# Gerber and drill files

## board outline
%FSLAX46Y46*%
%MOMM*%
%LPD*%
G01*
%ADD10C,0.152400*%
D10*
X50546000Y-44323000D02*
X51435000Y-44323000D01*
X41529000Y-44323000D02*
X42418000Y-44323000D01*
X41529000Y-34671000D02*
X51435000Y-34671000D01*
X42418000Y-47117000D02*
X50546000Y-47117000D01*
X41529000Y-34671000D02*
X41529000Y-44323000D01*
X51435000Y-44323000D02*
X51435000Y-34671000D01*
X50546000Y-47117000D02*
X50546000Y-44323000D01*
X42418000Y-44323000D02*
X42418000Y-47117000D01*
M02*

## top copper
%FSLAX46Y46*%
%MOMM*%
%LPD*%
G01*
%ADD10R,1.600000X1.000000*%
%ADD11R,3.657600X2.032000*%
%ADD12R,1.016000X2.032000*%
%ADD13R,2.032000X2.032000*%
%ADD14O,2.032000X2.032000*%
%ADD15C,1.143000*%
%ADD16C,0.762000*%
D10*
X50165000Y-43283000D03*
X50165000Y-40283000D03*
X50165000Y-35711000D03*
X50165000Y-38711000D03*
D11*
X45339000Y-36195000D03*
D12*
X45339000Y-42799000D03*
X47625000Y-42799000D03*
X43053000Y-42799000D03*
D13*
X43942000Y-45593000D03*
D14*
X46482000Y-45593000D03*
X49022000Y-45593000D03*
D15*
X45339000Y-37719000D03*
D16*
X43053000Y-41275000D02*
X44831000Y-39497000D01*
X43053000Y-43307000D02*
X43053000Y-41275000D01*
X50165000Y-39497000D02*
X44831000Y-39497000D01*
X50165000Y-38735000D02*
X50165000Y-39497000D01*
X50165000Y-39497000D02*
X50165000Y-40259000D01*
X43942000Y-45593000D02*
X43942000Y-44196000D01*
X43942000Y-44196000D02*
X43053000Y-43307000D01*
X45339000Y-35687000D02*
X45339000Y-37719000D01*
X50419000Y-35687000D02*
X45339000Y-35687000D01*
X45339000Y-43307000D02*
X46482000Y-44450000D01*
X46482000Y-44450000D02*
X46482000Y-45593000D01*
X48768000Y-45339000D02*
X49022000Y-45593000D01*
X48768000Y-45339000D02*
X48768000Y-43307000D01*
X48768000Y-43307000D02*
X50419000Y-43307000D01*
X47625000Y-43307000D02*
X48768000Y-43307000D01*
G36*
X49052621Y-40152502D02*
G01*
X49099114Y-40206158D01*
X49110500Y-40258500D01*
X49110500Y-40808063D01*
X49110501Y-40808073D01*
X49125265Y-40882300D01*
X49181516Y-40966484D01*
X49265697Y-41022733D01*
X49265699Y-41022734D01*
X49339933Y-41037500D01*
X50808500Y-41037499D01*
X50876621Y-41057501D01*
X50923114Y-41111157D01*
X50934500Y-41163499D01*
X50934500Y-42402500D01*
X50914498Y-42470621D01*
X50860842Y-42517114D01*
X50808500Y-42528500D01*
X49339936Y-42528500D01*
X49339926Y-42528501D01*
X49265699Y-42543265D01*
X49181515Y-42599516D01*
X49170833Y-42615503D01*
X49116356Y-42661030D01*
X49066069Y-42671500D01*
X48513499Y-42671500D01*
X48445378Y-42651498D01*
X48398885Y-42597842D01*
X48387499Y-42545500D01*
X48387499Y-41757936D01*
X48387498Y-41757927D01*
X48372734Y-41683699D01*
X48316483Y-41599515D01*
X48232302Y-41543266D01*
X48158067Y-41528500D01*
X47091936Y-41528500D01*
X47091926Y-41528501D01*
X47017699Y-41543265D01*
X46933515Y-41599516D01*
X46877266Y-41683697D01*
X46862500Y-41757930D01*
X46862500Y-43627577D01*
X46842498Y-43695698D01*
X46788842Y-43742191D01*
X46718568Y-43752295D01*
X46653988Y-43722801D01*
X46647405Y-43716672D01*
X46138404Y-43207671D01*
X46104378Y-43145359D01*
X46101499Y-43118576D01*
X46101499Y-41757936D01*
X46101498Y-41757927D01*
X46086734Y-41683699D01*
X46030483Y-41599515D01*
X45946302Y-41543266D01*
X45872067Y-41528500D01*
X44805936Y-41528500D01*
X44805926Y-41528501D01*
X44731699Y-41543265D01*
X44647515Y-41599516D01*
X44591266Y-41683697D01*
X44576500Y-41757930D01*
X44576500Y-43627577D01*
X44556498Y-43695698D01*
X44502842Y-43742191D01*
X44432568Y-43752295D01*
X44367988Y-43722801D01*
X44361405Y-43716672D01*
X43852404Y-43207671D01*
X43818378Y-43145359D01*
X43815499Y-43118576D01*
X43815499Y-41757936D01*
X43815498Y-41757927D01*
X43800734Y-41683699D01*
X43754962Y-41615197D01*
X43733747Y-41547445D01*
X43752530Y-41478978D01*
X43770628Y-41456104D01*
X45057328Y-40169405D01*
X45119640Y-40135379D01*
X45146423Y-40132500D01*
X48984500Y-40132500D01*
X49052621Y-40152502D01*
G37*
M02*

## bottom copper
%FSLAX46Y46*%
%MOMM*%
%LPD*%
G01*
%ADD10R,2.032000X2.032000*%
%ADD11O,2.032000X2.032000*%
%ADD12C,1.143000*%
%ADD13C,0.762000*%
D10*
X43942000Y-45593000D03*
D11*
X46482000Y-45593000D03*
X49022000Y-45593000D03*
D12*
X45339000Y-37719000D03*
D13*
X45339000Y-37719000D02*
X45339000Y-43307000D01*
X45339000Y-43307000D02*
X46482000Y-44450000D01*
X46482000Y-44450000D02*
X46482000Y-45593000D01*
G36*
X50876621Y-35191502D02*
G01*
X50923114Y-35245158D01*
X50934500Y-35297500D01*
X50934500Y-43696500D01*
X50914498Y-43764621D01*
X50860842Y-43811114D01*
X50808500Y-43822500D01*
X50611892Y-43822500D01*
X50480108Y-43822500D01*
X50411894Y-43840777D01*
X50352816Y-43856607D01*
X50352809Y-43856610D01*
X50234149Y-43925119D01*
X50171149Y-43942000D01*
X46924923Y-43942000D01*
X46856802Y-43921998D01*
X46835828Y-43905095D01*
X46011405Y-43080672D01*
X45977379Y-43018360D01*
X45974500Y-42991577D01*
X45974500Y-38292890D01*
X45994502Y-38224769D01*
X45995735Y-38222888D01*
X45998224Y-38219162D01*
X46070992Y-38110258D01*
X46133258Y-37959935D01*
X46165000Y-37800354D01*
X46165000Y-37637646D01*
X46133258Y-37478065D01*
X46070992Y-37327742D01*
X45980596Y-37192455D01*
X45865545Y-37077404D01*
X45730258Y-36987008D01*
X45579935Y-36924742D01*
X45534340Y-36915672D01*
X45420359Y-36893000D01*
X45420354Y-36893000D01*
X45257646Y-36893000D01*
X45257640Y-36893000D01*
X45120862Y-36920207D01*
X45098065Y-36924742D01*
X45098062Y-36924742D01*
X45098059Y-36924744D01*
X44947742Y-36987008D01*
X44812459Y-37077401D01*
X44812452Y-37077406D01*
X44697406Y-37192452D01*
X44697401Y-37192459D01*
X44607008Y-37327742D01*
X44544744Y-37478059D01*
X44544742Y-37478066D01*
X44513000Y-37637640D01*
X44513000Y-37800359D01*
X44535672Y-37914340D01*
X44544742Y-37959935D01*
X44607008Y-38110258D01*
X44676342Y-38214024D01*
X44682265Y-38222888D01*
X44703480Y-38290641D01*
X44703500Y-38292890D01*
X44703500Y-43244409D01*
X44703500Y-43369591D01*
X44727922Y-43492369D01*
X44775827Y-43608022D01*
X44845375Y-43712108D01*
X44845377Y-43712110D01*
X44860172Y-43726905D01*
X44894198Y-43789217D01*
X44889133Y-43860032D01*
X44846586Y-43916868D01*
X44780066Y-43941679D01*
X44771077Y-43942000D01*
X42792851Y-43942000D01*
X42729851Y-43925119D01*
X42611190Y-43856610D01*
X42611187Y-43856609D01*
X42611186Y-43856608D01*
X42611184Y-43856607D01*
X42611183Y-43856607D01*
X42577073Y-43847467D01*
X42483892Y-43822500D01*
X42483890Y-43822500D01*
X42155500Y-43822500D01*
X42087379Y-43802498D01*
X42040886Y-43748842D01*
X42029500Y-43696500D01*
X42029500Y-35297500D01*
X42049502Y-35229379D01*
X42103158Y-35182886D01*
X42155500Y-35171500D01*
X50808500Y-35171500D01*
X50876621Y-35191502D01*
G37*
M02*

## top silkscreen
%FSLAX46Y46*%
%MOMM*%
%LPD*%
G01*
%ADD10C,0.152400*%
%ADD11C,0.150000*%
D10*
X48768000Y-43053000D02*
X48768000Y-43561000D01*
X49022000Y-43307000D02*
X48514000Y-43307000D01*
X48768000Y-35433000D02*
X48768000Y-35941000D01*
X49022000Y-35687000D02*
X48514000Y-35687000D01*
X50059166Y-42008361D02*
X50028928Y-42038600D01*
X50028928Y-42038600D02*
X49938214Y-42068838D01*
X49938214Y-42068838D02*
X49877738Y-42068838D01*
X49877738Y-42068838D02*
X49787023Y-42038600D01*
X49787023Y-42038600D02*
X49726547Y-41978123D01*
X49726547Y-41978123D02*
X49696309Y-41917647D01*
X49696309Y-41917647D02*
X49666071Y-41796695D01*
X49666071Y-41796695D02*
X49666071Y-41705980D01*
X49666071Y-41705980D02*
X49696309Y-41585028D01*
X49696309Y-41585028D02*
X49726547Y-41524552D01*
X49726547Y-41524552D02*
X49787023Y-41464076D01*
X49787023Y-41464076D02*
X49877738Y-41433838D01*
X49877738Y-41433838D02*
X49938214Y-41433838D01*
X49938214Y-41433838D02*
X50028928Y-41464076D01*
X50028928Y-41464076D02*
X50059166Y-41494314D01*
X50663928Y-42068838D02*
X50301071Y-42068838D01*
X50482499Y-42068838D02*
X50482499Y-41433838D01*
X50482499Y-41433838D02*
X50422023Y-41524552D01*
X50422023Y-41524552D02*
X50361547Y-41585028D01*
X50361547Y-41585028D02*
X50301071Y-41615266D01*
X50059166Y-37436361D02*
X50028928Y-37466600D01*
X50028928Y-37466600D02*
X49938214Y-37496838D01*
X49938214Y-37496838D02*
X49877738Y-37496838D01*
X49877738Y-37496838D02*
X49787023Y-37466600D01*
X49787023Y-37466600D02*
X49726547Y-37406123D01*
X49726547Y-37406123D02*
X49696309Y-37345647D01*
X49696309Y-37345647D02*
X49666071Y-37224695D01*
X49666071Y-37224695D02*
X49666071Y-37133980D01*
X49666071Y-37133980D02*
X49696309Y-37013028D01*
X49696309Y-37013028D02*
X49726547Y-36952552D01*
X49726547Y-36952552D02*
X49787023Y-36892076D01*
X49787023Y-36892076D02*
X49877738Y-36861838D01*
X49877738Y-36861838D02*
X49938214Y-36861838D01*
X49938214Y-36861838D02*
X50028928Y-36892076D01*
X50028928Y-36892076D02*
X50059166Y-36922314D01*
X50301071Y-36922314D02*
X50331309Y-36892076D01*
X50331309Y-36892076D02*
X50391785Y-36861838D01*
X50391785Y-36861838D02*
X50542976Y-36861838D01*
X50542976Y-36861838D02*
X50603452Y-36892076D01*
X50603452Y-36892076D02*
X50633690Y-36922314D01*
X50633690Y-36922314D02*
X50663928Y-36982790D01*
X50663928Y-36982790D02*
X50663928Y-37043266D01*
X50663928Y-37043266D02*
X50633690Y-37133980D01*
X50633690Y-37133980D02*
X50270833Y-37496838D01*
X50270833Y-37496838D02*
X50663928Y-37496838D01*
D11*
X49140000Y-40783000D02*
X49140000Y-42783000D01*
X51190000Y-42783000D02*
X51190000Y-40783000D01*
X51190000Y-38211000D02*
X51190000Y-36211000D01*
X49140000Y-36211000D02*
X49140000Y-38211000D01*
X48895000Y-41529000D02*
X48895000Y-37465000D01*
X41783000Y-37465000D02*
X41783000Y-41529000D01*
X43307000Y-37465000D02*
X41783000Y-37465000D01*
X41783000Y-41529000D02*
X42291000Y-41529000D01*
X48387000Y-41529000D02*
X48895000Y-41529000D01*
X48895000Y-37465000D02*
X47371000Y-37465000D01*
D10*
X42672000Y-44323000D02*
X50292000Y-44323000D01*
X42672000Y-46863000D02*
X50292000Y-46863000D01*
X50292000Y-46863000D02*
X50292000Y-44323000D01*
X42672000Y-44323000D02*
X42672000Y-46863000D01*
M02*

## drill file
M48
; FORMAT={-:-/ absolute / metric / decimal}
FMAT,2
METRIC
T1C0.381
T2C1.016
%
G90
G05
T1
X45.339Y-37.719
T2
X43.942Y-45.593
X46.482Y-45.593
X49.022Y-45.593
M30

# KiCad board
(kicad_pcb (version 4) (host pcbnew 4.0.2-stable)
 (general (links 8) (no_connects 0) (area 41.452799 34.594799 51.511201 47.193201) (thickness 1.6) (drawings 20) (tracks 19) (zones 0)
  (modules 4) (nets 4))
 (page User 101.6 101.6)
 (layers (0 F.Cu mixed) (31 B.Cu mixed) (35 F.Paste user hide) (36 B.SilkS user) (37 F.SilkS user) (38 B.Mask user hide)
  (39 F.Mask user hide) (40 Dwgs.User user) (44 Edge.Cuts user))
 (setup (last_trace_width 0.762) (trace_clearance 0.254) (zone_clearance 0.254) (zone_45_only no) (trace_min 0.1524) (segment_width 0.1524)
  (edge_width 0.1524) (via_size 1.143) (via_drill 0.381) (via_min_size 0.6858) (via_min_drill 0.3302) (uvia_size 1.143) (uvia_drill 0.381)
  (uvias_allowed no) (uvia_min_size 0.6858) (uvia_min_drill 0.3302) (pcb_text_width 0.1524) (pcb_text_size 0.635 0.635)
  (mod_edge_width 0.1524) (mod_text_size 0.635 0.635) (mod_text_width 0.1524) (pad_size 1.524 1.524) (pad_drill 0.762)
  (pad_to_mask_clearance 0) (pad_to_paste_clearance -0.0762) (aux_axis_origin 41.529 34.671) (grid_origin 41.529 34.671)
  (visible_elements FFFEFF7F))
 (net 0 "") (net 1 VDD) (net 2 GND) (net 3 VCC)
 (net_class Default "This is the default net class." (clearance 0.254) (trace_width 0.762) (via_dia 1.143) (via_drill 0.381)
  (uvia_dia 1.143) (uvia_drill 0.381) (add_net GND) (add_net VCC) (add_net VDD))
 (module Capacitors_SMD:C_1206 (layer F.Cu) (at 50.165 41.783 90)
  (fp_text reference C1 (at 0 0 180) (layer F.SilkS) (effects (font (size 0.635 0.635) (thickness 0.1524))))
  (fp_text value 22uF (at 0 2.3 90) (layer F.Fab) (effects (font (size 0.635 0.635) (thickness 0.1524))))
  (fp_line (start 1 -1.025) (end -1 -1.025) (layer F.SilkS) (width 0.15))
  (fp_line (start -1 1.025) (end 1 1.025) (layer F.SilkS) (width 0.15))
  (pad 1 smd rect (at -1.5 0 90) (size 1 1.6) (layers F.Cu F.Paste F.Mask) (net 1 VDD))
  (pad 2 smd rect (at 1.5 0 90) (size 1 1.6) (layers F.Cu F.Paste F.Mask) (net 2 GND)))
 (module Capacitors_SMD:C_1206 (layer F.Cu) (at 50.165 37.211 270)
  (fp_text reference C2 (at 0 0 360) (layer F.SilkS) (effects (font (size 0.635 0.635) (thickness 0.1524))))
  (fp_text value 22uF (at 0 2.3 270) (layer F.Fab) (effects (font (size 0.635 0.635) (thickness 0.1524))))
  (fp_line (start 1 -1.025) (end -1 -1.025) (layer F.SilkS) (width 0.15))
  (fp_line (start -1 1.025) (end 1 1.025) (layer F.SilkS) (width 0.15))
  (pad 1 smd rect (at -1.5 0 270) (size 1 1.6) (layers F.Cu F.Paste F.Mask) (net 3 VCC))
  (pad 2 smd rect (at 1.5 0 270) (size 1 1.6) (layers F.Cu F.Paste F.Mask) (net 2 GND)))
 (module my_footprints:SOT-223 (layer F.Cu) (at 45.339 39.497)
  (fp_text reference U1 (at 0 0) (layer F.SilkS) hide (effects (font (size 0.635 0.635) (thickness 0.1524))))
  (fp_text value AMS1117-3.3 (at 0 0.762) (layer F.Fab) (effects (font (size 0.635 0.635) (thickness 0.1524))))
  (fp_line (start 3.556 2.032) (end 3.556 -2.032) (layer F.SilkS) (width 0.15))
  (fp_line (start -3.556 -2.032) (end -3.556 2.032) (layer F.SilkS) (width 0.15))
  (fp_line (start -2.032 -2.032) (end -3.556 -2.032) (layer F.SilkS) (width 0.15))
  (fp_line (start -3.556 2.032) (end -3.048 2.032) (layer F.SilkS) (width 0.15))
  (fp_line (start 3.048 2.032) (end 3.556 2.032) (layer F.SilkS) (width 0.15))
  (fp_line (start 3.556 -2.032) (end 2.032 -2.032) (layer F.SilkS) (width 0.15))
  (pad 4 smd rect (at 0 -3.302) (size 3.6576 2.032) (layers F.Cu F.Paste F.Mask) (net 3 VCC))
  (pad 2 smd rect (at 0 3.302) (size 1.016 2.032) (layers F.Cu F.Paste F.Mask) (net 3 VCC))
  (pad 3 smd rect (at 2.286 3.302) (size 1.016 2.032) (layers F.Cu F.Paste F.Mask) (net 1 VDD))
  (pad 1 smd rect (at -2.286 3.302) (size 1.016 2.032) (layers F.Cu F.Paste F.Mask) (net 2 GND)))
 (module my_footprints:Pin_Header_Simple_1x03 (layer F.Cu) (at 43.942 45.593 90)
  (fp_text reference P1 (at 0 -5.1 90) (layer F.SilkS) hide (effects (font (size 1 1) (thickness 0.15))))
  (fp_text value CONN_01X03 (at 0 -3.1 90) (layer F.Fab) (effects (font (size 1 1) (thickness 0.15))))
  (fp_line (start 1.27 -1.27) (end 1.27 6.35) (layer F.SilkS) (width 0.1524))
  (fp_line (start -1.27 -1.27) (end -1.27 6.35) (layer F.SilkS) (width 0.1524))
  (fp_line (start -1.27 6.35) (end 1.27 6.35) (layer F.SilkS) (width 0.1524))
  (fp_line (start 1.27 -1.27) (end -1.27 -1.27) (layer F.SilkS) (width 0.1524))
  (pad 1 thru_hole rect (at 0 0 90) (size 2.032 2.032) (drill 1.016) (layers *.Cu *.Mask) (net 2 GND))
  (pad 2 thru_hole oval (at 0 2.54 90) (size 2.032 2.032) (drill 1.016) (layers *.Cu *.Mask) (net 3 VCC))
  (pad 3 thru_hole oval (at 0 5.08 90) (size 2.032 2.032) (drill 1.016) (layers *.Cu *.Mask) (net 1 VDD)))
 (gr_line (start 50.546 44.323) (end 51.435 44.323) (angle 90) (layer Edge.Cuts) (width 0.1524))
 (gr_line (start 41.529 44.323) (end 42.418 44.323) (angle 90) (layer Edge.Cuts) (width 0.1524))
 (gr_line (start 41.529 34.671) (end 51.435 34.671) (angle 90) (layer Edge.Cuts) (width 0.1524))
 (gr_line (start 48.768 43.053) (end 48.768 43.561) (angle 90) (layer F.SilkS) (width 0.1524))
 (gr_line (start 49.022 43.307) (end 48.514 43.307) (angle 90) (layer F.SilkS) (width 0.1524))
 (gr_line (start 48.768 35.433) (end 48.768 35.941) (angle 90) (layer F.SilkS) (width 0.1524))
 (gr_line (start 49.022 35.687) (end 48.514 35.687) (angle 90) (layer F.SilkS) (width 0.1524))
 (gr_line (start 42.418 47.117) (end 50.546 47.117) (angle 90) (layer Edge.Cuts) (width 0.1524))
 (gr_line (start 41.529 34.671) (end 41.529 44.323) (angle 90) (layer Edge.Cuts) (width 0.1524))
 (gr_line (start 51.435 44.323) (end 51.435 34.671) (angle 90) (layer Edge.Cuts) (width 0.1524))
 (gr_line (start 50.546 47.117) (end 50.546 44.323) (angle 90) (layer Edge.Cuts) (width 0.1524))
 (gr_line (start 42.418 44.323) (end 42.418 47.117) (angle 90) (layer Edge.Cuts) (width 0.1524))
 (segment (start 43.053 41.275) (end 44.831 39.497) (width 0.762) (layer F.Cu) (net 2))
 (segment (start 43.053 43.307) (end 43.053 41.275) (width 0.762) (layer F.Cu) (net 2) (status 30))
 (segment (start 50.165 39.497) (end 44.831 39.497) (width 0.762) (layer F.Cu) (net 2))
 (segment (start 50.165 38.735) (end 50.165 39.497) (width 0.762) (layer F.Cu) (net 2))
 (segment (start 50.165 39.497) (end 50.165 40.259) (width 0.762) (layer F.Cu) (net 2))
 (segment (start 43.942 45.593) (end 43.942 44.196) (width 0.762) (layer F.Cu) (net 2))
 (segment (start 43.942 44.196) (end 43.053 43.307) (width 0.762) (layer F.Cu) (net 2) (status 20))
 (segment (start 45.339 35.687) (end 45.339 37.719) (width 0.762) (layer F.Cu) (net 3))
 (via (at 45.339 37.719) (size 1.143) (drill 0.381) (layers F.Cu B.Cu) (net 3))
 (segment (start 45.339 37.719) (end 45.339 43.307) (width 0.762) (layer B.Cu) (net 3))
 (segment (start 45.339 43.307) (end 46.482 44.45) (width 0.762) (layer B.Cu) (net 3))
 (segment (start 46.482 44.45) (end 46.482 45.593) (width 0.762) (layer B.Cu) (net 3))
 (segment (start 50.419 35.687) (end 45.339 35.687) (width 0.762) (layer F.Cu) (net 3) (status 20))
 (segment (start 45.339 43.307) (end 46.482 44.45) (width 0.762) (layer F.Cu) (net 3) (status 10))
 (segment (start 46.482 44.45) (end 46.482 45.593) (width 0.762) (layer F.Cu) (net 3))
 (segment (start 48.768 45.339) (end 49.022 45.593) (width 0.762) (layer F.Cu) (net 1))
 (segment (start 48.768 45.339) (end 48.768 43.307) (width 0.762) (layer F.Cu) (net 1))
 (segment (start 48.768 43.307) (end 50.419 43.307) (width 0.762) (layer F.Cu) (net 1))
 (segment (start 47.625 43.307) (end 48.768 43.307) (width 0.762) (layer F.Cu) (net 1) (status 10))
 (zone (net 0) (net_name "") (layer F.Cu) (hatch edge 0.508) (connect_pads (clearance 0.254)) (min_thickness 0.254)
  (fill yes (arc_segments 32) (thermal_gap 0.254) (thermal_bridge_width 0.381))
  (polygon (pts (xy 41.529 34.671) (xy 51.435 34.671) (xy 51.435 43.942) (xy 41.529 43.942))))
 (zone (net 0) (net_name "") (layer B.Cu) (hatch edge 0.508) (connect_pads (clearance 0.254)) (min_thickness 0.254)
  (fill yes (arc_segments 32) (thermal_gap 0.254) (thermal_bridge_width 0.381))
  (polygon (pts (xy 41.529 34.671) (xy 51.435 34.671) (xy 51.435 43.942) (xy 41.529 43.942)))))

